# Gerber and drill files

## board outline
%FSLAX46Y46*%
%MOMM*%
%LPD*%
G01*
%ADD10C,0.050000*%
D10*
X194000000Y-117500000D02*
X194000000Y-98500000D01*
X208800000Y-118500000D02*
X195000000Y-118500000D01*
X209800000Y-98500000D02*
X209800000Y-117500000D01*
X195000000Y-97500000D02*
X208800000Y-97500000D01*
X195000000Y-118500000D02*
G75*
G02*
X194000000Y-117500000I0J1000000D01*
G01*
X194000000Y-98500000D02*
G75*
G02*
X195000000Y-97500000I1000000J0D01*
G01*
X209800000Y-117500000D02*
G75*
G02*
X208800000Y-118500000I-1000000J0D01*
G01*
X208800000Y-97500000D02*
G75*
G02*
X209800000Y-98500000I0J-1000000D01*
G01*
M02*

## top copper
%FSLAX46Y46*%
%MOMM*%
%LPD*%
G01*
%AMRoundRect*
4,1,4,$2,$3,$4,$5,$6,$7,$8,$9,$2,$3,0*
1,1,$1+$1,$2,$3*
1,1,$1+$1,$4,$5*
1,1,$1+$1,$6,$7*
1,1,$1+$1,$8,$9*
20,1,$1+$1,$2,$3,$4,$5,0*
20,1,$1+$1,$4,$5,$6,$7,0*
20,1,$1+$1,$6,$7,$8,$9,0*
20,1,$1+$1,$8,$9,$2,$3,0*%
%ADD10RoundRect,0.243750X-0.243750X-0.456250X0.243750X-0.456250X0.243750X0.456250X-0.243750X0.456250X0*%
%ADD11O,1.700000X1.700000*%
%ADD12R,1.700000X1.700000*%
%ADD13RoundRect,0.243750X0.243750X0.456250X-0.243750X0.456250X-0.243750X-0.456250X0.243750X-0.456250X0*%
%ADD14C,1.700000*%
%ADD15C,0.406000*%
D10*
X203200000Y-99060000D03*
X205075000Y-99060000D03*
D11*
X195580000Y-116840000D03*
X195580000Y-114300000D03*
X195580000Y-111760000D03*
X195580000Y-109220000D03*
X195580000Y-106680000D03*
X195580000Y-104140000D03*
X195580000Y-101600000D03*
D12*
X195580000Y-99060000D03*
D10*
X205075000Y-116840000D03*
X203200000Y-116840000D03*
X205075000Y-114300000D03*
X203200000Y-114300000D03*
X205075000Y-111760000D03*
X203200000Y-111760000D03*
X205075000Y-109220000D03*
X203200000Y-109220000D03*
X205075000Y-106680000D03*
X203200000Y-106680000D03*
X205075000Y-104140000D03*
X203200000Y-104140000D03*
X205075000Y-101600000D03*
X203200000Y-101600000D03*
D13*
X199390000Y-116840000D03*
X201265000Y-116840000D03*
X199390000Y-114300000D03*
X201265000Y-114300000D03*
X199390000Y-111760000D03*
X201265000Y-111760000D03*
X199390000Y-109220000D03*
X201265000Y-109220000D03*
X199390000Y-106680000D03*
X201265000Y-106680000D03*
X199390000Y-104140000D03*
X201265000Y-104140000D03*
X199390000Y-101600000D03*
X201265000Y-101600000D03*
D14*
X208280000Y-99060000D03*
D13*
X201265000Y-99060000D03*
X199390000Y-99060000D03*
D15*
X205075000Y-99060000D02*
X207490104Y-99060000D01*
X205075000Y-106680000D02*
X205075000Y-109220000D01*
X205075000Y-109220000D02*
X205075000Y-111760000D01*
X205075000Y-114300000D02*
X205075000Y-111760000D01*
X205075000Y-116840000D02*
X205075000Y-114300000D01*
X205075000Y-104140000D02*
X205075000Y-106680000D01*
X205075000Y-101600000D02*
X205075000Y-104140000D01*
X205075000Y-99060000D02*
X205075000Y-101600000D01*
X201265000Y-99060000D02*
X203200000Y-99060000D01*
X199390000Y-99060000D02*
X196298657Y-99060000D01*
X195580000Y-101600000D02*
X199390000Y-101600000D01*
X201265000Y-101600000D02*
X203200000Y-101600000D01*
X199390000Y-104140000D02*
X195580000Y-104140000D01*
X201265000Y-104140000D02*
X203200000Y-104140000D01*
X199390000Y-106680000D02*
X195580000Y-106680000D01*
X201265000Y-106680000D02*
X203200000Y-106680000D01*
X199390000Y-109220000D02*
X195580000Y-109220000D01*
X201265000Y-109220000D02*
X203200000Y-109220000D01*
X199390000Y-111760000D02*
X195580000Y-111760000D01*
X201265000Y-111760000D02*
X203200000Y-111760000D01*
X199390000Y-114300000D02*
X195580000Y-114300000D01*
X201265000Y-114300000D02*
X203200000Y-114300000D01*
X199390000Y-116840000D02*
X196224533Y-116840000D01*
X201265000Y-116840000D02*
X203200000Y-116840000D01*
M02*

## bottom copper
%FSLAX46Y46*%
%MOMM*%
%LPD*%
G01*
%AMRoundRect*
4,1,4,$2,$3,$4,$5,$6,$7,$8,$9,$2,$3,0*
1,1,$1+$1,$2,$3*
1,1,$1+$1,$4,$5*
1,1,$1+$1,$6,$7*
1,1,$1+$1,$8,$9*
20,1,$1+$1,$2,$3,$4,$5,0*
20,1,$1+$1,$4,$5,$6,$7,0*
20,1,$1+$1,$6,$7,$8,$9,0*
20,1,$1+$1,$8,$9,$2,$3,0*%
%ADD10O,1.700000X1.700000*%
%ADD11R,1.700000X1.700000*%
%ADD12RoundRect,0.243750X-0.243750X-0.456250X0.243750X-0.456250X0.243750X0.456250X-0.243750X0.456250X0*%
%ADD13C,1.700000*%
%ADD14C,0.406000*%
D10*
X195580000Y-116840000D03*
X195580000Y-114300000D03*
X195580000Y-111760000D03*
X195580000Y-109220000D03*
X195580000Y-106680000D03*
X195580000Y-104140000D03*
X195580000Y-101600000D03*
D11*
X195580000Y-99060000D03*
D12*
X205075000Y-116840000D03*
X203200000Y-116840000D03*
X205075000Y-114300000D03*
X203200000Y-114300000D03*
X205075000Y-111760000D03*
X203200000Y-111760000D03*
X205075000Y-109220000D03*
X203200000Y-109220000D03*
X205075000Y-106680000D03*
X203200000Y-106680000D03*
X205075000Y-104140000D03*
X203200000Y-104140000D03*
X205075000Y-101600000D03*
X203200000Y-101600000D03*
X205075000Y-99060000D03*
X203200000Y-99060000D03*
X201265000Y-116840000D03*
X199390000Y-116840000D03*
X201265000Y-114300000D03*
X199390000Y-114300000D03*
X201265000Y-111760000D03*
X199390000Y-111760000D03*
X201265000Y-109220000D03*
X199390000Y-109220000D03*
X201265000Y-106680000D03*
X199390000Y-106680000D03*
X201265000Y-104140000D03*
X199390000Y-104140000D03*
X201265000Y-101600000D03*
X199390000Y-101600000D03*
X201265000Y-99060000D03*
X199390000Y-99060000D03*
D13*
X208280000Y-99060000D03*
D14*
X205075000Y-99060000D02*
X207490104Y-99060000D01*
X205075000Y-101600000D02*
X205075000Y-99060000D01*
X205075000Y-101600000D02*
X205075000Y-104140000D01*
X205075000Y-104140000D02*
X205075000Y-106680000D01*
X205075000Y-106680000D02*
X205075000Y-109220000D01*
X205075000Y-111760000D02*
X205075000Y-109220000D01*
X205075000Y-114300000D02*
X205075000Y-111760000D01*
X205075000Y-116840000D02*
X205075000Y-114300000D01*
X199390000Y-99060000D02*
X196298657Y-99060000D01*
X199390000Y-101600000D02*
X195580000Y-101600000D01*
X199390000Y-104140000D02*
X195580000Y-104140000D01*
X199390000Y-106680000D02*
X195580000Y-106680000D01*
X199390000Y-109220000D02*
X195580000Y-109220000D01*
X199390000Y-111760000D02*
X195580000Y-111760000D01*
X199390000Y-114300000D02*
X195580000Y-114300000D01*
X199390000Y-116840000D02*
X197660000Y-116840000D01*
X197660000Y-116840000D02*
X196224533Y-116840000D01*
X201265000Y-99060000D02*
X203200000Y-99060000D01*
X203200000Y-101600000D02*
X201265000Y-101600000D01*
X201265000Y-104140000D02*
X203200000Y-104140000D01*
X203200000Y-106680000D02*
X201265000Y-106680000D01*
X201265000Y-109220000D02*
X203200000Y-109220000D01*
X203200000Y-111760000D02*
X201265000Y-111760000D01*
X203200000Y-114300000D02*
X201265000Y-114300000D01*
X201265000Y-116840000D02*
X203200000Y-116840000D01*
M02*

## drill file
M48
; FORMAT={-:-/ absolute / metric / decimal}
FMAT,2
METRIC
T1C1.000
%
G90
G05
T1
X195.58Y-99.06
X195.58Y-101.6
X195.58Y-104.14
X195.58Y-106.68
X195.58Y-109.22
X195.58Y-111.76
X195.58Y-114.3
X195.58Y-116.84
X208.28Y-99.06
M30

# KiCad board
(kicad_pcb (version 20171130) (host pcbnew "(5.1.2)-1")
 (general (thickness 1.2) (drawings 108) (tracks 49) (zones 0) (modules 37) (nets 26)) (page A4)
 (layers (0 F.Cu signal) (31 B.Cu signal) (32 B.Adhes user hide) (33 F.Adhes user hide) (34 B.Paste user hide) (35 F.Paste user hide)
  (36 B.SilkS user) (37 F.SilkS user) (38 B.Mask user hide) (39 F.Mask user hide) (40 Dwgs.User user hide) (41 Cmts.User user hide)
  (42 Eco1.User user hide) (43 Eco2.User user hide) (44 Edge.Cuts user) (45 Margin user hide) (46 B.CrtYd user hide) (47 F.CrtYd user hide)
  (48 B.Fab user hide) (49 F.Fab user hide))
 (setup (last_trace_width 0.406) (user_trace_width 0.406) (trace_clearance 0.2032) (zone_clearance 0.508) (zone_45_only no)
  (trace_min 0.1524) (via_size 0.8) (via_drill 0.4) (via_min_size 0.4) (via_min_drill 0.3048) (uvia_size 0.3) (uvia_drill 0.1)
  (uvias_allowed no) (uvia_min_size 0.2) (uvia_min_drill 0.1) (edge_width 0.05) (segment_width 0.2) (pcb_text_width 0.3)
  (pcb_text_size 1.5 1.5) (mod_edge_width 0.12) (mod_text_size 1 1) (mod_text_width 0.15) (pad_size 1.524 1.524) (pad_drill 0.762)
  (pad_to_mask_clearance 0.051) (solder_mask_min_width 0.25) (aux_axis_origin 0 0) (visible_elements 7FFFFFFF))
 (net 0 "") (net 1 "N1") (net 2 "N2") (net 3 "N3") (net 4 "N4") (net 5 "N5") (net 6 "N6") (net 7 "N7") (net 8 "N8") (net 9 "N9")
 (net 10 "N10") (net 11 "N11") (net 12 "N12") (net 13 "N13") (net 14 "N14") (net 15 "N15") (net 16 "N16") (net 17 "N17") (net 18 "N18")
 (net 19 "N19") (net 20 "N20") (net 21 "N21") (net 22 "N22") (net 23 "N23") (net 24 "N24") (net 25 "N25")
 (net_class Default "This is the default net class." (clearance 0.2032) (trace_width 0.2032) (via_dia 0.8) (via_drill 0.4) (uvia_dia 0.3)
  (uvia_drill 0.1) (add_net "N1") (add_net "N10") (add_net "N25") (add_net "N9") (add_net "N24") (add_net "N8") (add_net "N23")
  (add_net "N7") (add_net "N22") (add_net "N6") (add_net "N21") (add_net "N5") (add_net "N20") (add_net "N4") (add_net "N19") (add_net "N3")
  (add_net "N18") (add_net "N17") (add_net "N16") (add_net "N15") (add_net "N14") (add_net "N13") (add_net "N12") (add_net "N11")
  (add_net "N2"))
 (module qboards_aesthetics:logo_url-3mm (layer F.Cu) (at 208.026 116.332 90)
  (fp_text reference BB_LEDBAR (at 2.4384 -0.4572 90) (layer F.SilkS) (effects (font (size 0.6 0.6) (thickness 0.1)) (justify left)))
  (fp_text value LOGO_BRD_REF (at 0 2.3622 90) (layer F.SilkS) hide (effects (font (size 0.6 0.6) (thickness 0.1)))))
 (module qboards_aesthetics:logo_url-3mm (layer B.Cu) (at 208.026 107.442 270)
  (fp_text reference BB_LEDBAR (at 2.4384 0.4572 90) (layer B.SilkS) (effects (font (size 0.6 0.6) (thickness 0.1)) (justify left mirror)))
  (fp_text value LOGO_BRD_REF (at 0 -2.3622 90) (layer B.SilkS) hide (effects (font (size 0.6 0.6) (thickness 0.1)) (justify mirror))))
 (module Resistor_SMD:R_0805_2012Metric (layer F.Cu) (at 204.1375 99.06)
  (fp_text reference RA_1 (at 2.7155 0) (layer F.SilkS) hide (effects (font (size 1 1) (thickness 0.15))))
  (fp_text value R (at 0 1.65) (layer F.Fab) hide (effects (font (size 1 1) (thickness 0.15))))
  (pad 1 smd roundrect (at -0.9375 0) (size 0.975 1.4) (layers F.Cu F.Paste F.Mask) (roundrect_rratio 0.25) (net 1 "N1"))
  (pad 2 smd roundrect (at 0.9375 0) (size 0.975 1.4) (layers F.Cu F.Paste F.Mask) (roundrect_rratio 0.25) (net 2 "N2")))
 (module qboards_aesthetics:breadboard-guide (layer F.Cu) (at 162.56 96.52)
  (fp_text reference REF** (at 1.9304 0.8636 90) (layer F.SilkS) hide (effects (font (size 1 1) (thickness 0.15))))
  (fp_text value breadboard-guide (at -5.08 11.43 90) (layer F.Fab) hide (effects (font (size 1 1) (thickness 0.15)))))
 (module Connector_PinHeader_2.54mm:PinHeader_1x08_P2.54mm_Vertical (layer B.Cu) (at 195.58 99.06 180)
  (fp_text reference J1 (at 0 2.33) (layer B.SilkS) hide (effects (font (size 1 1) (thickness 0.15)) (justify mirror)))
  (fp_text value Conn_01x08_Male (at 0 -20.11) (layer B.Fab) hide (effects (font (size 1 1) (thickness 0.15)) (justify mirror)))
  (pad 8 thru_hole oval (at 0 -17.78 180) (size 1.7 1.7) (drill 1) (layers *.Cu *.Mask) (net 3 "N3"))
  (pad 7 thru_hole oval (at 0 -15.24 180) (size 1.7 1.7) (drill 1) (layers *.Cu *.Mask) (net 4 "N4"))
  (pad 6 thru_hole oval (at 0 -12.7 180) (size 1.7 1.7) (drill 1) (layers *.Cu *.Mask) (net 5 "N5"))
  (pad 5 thru_hole oval (at 0 -10.16 180) (size 1.7 1.7) (drill 1) (layers *.Cu *.Mask) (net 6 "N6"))
  (pad 4 thru_hole oval (at 0 -7.62 180) (size 1.7 1.7) (drill 1) (layers *.Cu *.Mask) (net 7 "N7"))
  (pad 3 thru_hole oval (at 0 -5.08 180) (size 1.7 1.7) (drill 1) (layers *.Cu *.Mask) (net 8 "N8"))
  (pad 2 thru_hole oval (at 0 -2.54 180) (size 1.7 1.7) (drill 1) (layers *.Cu *.Mask) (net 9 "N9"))
  (pad 1 thru_hole rect (at 0 0 180) (size 1.7 1.7) (drill 1) (layers *.Cu *.Mask) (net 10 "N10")))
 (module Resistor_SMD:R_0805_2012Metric (layer B.Cu) (at 204.1375 116.84)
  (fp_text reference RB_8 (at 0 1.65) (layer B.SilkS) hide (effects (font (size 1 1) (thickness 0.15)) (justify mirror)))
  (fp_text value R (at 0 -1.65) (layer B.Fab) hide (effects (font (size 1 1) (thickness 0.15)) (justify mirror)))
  (pad 2 smd roundrect (at 0.9375 0) (size 0.975 1.4) (layers B.Cu B.Paste B.Mask) (roundrect_rratio 0.25) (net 2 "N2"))
  (pad 1 smd roundrect (at -0.9375 0) (size 0.975 1.4) (layers B.Cu B.Paste B.Mask) (roundrect_rratio 0.25) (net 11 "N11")))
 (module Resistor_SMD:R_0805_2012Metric (layer B.Cu) (at 204.1375 114.3)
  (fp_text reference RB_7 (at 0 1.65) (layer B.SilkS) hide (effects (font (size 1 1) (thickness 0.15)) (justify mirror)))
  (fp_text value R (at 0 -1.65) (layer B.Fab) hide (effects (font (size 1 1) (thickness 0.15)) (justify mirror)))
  (pad 2 smd roundrect (at 0.9375 0) (size 0.975 1.4) (layers B.Cu B.Paste B.Mask) (roundrect_rratio 0.25) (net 2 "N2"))
  (pad 1 smd roundrect (at -0.9375 0) (size 0.975 1.4) (layers B.Cu B.Paste B.Mask) (roundrect_rratio 0.25) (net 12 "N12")))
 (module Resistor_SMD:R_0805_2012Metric (layer B.Cu) (at 204.1375 111.76)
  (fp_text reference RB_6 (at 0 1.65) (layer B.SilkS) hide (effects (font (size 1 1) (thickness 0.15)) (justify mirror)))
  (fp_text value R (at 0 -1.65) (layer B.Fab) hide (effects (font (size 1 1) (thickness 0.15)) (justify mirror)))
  (pad 2 smd roundrect (at 0.9375 0) (size 0.975 1.4) (layers B.Cu B.Paste B.Mask) (roundrect_rratio 0.25) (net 2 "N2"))
  (pad 1 smd roundrect (at -0.9375 0) (size 0.975 1.4) (layers B.Cu B.Paste B.Mask) (roundrect_rratio 0.25) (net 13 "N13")))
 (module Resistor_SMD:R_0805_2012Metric (layer B.Cu) (at 204.1375 109.22)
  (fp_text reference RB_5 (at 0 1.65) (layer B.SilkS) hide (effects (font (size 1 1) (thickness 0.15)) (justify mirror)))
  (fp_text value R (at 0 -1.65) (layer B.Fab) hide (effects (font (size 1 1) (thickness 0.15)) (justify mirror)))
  (pad 2 smd roundrect (at 0.9375 0) (size 0.975 1.4) (layers B.Cu B.Paste B.Mask) (roundrect_rratio 0.25) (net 2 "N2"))
  (pad 1 smd roundrect (at -0.9375 0) (size 0.975 1.4) (layers B.Cu B.Paste B.Mask) (roundrect_rratio 0.25) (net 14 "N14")))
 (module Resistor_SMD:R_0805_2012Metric (layer B.Cu) (at 204.1375 106.68)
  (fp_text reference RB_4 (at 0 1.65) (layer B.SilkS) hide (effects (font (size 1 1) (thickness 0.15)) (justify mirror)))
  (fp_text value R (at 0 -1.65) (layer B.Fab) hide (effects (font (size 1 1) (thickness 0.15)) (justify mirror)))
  (pad 2 smd roundrect (at 0.9375 0) (size 0.975 1.4) (layers B.Cu B.Paste B.Mask) (roundrect_rratio 0.25) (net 2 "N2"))
  (pad 1 smd roundrect (at -0.9375 0) (size 0.975 1.4) (layers B.Cu B.Paste B.Mask) (roundrect_rratio 0.25) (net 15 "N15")))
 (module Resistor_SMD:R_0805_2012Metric (layer B.Cu) (at 204.1375 104.14)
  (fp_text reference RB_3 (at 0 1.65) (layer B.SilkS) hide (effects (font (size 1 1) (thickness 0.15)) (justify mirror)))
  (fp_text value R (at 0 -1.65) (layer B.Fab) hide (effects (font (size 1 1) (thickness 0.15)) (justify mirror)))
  (pad 2 smd roundrect (at 0.9375 0) (size 0.975 1.4) (layers B.Cu B.Paste B.Mask) (roundrect_rratio 0.25) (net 2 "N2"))
  (pad 1 smd roundrect (at -0.9375 0) (size 0.975 1.4) (layers B.Cu B.Paste B.Mask) (roundrect_rratio 0.25) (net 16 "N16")))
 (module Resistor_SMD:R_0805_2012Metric (layer B.Cu) (at 204.1375 101.6)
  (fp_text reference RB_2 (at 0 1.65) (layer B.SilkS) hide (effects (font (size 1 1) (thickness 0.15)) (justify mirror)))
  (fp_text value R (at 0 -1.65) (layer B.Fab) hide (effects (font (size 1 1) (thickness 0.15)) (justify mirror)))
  (pad 2 smd roundrect (at 0.9375 0) (size 0.975 1.4) (layers B.Cu B.Paste B.Mask) (roundrect_rratio 0.25) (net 2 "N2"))
  (pad 1 smd roundrect (at -0.9375 0) (size 0.975 1.4) (layers B.Cu B.Paste B.Mask) (roundrect_rratio 0.25) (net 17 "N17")))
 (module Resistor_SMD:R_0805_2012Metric (layer B.Cu) (at 204.1375 99.06)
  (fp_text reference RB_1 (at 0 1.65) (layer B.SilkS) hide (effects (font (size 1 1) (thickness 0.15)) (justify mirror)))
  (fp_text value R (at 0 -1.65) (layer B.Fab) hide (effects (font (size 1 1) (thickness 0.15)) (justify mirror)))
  (pad 2 smd roundrect (at 0.9375 0) (size 0.975 1.4) (layers B.Cu B.Paste B.Mask) (roundrect_rratio 0.25) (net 2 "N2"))
  (pad 1 smd roundrect (at -0.9375 0) (size 0.975 1.4) (layers B.Cu B.Paste B.Mask) (roundrect_rratio 0.25) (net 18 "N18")))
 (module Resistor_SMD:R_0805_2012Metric (layer F.Cu) (at 204.1375 116.84)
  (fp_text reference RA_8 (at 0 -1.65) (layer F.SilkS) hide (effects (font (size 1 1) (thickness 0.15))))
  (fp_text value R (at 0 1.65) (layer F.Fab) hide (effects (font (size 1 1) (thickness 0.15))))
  (pad 2 smd roundrect (at 0.9375 0) (size 0.975 1.4) (layers F.Cu F.Paste F.Mask) (roundrect_rratio 0.25) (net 2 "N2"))
  (pad 1 smd roundrect (at -0.9375 0) (size 0.975 1.4) (layers F.Cu F.Paste F.Mask) (roundrect_rratio 0.25) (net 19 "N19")))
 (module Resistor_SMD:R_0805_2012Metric (layer F.Cu) (at 204.1375 114.3)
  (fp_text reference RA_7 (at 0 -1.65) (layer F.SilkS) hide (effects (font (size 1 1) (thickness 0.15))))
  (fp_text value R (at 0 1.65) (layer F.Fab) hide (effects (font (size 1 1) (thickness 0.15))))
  (pad 2 smd roundrect (at 0.9375 0) (size 0.975 1.4) (layers F.Cu F.Paste F.Mask) (roundrect_rratio 0.25) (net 2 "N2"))
  (pad 1 smd roundrect (at -0.9375 0) (size 0.975 1.4) (layers F.Cu F.Paste F.Mask) (roundrect_rratio 0.25) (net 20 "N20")))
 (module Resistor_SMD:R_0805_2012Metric (layer F.Cu) (at 204.1375 111.76)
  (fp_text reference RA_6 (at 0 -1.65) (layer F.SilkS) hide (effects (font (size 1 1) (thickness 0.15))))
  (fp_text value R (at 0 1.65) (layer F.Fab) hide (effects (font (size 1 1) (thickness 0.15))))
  (pad 2 smd roundrect (at 0.9375 0) (size 0.975 1.4) (layers F.Cu F.Paste F.Mask) (roundrect_rratio 0.25) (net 2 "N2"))
  (pad 1 smd roundrect (at -0.9375 0) (size 0.975 1.4) (layers F.Cu F.Paste F.Mask) (roundrect_rratio 0.25) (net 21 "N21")))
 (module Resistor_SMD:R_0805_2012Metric (layer F.Cu) (at 204.1375 109.22)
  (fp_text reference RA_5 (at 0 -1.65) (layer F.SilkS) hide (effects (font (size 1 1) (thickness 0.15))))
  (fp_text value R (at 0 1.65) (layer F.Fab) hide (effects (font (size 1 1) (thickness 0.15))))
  (pad 2 smd roundrect (at 0.9375 0) (size 0.975 1.4) (layers F.Cu F.Paste F.Mask) (roundrect_rratio 0.25) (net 2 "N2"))
  (pad 1 smd roundrect (at -0.9375 0) (size 0.975 1.4) (layers F.Cu F.Paste F.Mask) (roundrect_rratio 0.25) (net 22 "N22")))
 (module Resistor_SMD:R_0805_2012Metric (layer F.Cu) (at 204.1375 106.68)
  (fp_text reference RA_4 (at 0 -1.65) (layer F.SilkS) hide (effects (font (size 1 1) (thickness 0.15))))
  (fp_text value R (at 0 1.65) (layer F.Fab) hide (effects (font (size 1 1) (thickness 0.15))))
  (pad 2 smd roundrect (at 0.9375 0) (size 0.975 1.4) (layers F.Cu F.Paste F.Mask) (roundrect_rratio 0.25) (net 2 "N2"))
  (pad 1 smd roundrect (at -0.9375 0) (size 0.975 1.4) (layers F.Cu F.Paste F.Mask) (roundrect_rratio 0.25) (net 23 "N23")))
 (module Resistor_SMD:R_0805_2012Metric (layer F.Cu) (at 204.1375 104.14)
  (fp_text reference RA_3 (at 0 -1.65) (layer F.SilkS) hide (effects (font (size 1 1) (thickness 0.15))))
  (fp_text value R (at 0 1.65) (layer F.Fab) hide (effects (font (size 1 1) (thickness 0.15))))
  (pad 2 smd roundrect (at 0.9375 0) (size 0.975 1.4) (layers F.Cu F.Paste F.Mask) (roundrect_rratio 0.25) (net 2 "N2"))
  (pad 1 smd roundrect (at -0.9375 0) (size 0.975 1.4) (layers F.Cu F.Paste F.Mask) (roundrect_rratio 0.25) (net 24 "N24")))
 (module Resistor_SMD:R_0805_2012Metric (layer F.Cu) (at 204.1375 101.6)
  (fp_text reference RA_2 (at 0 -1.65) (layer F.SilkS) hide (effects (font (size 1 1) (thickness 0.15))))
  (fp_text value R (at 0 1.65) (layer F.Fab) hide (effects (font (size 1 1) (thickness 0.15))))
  (pad 2 smd roundrect (at 0.9375 0) (size 0.975 1.4) (layers F.Cu F.Paste F.Mask) (roundrect_rratio 0.25) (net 2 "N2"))
  (pad 1 smd roundrect (at -0.9375 0) (size 0.975 1.4) (layers F.Cu F.Paste F.Mask) (roundrect_rratio 0.25) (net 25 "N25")))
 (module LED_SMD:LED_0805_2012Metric (layer B.Cu) (at 200.3275 116.84)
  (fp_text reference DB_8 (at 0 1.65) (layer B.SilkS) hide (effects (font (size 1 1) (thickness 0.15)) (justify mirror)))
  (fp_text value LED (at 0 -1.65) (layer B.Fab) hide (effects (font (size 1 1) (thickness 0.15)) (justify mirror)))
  (pad 2 smd roundrect (at 0.9375 0) (size 0.975 1.4) (layers B.Cu B.Paste B.Mask) (roundrect_rratio 0.25) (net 11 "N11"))
  (pad 1 smd roundrect (at -0.9375 0) (size 0.975 1.4) (layers B.Cu B.Paste B.Mask) (roundrect_rratio 0.25) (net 3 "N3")))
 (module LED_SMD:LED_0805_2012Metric (layer B.Cu) (at 200.3275 114.3)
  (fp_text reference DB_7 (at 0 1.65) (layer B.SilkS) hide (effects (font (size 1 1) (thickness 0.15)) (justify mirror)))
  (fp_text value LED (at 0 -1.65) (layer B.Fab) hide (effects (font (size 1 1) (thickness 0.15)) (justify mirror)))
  (pad 2 smd roundrect (at 0.9375 0) (size 0.975 1.4) (layers B.Cu B.Paste B.Mask) (roundrect_rratio 0.25) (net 12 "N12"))
  (pad 1 smd roundrect (at -0.9375 0) (size 0.975 1.4) (layers B.Cu B.Paste B.Mask) (roundrect_rratio 0.25) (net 4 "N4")))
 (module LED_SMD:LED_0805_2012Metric (layer B.Cu) (at 200.3275 111.76)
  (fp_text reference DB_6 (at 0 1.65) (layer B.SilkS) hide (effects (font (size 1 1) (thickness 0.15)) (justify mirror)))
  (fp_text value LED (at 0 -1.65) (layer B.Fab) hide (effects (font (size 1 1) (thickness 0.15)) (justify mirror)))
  (pad 2 smd roundrect (at 0.9375 0) (size 0.975 1.4) (layers B.Cu B.Paste B.Mask) (roundrect_rratio 0.25) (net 13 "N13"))
  (pad 1 smd roundrect (at -0.9375 0) (size 0.975 1.4) (layers B.Cu B.Paste B.Mask) (roundrect_rratio 0.25) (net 5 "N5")))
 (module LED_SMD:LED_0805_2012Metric (layer B.Cu) (at 200.3275 109.22)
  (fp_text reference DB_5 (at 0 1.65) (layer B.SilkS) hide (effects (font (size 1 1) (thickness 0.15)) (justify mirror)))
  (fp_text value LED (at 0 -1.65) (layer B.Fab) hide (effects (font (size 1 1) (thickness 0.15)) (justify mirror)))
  (pad 2 smd roundrect (at 0.9375 0) (size 0.975 1.4) (layers B.Cu B.Paste B.Mask) (roundrect_rratio 0.25) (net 14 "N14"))
  (pad 1 smd roundrect (at -0.9375 0) (size 0.975 1.4) (layers B.Cu B.Paste B.Mask) (roundrect_rratio 0.25) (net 6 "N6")))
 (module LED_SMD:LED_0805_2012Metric (layer B.Cu) (at 200.3275 106.68)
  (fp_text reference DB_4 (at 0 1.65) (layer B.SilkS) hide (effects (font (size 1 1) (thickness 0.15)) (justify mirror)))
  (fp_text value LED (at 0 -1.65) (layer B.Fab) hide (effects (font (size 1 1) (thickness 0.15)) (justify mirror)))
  (pad 2 smd roundrect (at 0.9375 0) (size 0.975 1.4) (layers B.Cu B.Paste B.Mask) (roundrect_rratio 0.25) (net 15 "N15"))
  (pad 1 smd roundrect (at -0.9375 0) (size 0.975 1.4) (layers B.Cu B.Paste B.Mask) (roundrect_rratio 0.25) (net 7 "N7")))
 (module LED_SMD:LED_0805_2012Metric (layer B.Cu) (at 200.3275 104.14)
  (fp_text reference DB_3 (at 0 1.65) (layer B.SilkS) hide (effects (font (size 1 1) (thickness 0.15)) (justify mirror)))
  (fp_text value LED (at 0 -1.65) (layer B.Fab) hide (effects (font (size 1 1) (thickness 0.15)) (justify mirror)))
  (pad 2 smd roundrect (at 0.9375 0) (size 0.975 1.4) (layers B.Cu B.Paste B.Mask) (roundrect_rratio 0.25) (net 16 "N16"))
  (pad 1 smd roundrect (at -0.9375 0) (size 0.975 1.4) (layers B.Cu B.Paste B.Mask) (roundrect_rratio 0.25) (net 8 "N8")))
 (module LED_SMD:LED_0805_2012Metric (layer B.Cu) (at 200.3275 101.6)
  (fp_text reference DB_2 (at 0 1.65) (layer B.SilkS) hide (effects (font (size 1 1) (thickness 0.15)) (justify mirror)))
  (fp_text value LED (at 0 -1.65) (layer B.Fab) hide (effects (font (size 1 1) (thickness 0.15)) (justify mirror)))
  (pad 2 smd roundrect (at 0.9375 0) (size 0.975 1.4) (layers B.Cu B.Paste B.Mask) (roundrect_rratio 0.25) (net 17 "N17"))
  (pad 1 smd roundrect (at -0.9375 0) (size 0.975 1.4) (layers B.Cu B.Paste B.Mask) (roundrect_rratio 0.25) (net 9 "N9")))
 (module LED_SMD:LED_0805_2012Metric (layer B.Cu) (at 200.3275 99.06)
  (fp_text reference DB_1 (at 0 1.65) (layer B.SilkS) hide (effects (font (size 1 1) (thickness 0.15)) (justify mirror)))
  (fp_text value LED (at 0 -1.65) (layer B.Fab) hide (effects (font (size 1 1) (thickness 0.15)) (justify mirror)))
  (pad 2 smd roundrect (at 0.9375 0) (size 0.975 1.4) (layers B.Cu B.Paste B.Mask) (roundrect_rratio 0.25) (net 18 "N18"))
  (pad 1 smd roundrect (at -0.9375 0) (size 0.975 1.4) (layers B.Cu B.Paste B.Mask) (roundrect_rratio 0.25) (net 10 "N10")))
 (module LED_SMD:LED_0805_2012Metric (layer F.Cu) (at 200.3275 116.84 180)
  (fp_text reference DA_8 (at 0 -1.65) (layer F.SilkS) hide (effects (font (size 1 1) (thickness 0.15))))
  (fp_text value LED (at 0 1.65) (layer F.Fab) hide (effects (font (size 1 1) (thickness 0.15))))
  (pad 2 smd roundrect (at 0.9375 0 180) (size 0.975 1.4) (layers F.Cu F.Paste F.Mask) (roundrect_rratio 0.25) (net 3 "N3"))
  (pad 1 smd roundrect (at -0.9375 0 180) (size 0.975 1.4) (layers F.Cu F.Paste F.Mask) (roundrect_rratio 0.25) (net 19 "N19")))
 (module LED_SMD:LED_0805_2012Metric (layer F.Cu) (at 200.3275 114.3 180)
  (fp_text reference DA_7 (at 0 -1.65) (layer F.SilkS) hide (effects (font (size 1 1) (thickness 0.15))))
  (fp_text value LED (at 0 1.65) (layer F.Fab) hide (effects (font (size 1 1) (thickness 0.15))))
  (pad 2 smd roundrect (at 0.9375 0 180) (size 0.975 1.4) (layers F.Cu F.Paste F.Mask) (roundrect_rratio 0.25) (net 4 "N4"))
  (pad 1 smd roundrect (at -0.9375 0 180) (size 0.975 1.4) (layers F.Cu F.Paste F.Mask) (roundrect_rratio 0.25) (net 20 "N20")))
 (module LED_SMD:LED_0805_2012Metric (layer F.Cu) (at 200.3275 111.76 180)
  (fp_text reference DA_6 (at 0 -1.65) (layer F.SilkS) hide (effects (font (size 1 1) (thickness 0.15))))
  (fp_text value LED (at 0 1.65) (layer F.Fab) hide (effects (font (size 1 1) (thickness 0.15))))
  (pad 2 smd roundrect (at 0.9375 0 180) (size 0.975 1.4) (layers F.Cu F.Paste F.Mask) (roundrect_rratio 0.25) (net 5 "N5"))
  (pad 1 smd roundrect (at -0.9375 0 180) (size 0.975 1.4) (layers F.Cu F.Paste F.Mask) (roundrect_rratio 0.25) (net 21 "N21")))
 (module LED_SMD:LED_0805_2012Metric (layer F.Cu) (at 200.3275 109.22 180)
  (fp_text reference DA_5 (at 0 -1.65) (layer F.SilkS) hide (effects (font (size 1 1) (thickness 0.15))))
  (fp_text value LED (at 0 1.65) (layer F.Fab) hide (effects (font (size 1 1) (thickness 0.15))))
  (pad 2 smd roundrect (at 0.9375 0 180) (size 0.975 1.4) (layers F.Cu F.Paste F.Mask) (roundrect_rratio 0.25) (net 6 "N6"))
  (pad 1 smd roundrect (at -0.9375 0 180) (size 0.975 1.4) (layers F.Cu F.Paste F.Mask) (roundrect_rratio 0.25) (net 22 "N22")))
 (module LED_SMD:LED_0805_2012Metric (layer F.Cu) (at 200.3275 106.68 180)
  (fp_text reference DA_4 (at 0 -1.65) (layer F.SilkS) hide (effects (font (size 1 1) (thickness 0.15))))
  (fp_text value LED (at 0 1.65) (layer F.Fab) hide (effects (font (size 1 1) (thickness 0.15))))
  (pad 2 smd roundrect (at 0.9375 0 180) (size 0.975 1.4) (layers F.Cu F.Paste F.Mask) (roundrect_rratio 0.25) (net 7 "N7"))
  (pad 1 smd roundrect (at -0.9375 0 180) (size 0.975 1.4) (layers F.Cu F.Paste F.Mask) (roundrect_rratio 0.25) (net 23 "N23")))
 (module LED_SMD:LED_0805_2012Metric (layer F.Cu) (at 200.3275 104.14 180)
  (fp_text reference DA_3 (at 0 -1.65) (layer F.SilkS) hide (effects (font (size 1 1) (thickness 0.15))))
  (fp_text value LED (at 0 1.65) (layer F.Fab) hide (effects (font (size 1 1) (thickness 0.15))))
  (pad 2 smd roundrect (at 0.9375 0 180) (size 0.975 1.4) (layers F.Cu F.Paste F.Mask) (roundrect_rratio 0.25) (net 8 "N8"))
  (pad 1 smd roundrect (at -0.9375 0 180) (size 0.975 1.4) (layers F.Cu F.Paste F.Mask) (roundrect_rratio 0.25) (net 24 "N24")))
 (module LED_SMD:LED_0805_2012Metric (layer F.Cu) (at 200.3275 101.6 180)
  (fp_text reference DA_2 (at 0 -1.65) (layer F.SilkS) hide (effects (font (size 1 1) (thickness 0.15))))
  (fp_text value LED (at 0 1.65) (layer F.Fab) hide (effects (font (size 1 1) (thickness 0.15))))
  (pad 2 smd roundrect (at 0.9375 0 180) (size 0.975 1.4) (layers F.Cu F.Paste F.Mask) (roundrect_rratio 0.25) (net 9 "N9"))
  (pad 1 smd roundrect (at -0.9375 0 180) (size 0.975 1.4) (layers F.Cu F.Paste F.Mask) (roundrect_rratio 0.25) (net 25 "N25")))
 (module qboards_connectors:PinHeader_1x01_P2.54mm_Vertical (layer F.Cu) (at 208.28 99.06 90)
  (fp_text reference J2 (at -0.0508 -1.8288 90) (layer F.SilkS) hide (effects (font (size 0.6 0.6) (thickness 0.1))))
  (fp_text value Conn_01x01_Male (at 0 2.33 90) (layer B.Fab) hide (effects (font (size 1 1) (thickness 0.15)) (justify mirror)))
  (pad 1 thru_hole circle (at 0 0 90) (size 1.7 1.7) (drill 1) (layers *.Cu *.Mask) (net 2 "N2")))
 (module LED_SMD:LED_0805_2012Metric (layer F.Cu) (at 200.3275 99.06 180)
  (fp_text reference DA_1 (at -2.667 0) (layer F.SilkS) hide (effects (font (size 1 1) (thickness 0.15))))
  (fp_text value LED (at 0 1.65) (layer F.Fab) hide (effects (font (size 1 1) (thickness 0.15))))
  (pad 1 smd roundrect (at -0.9375 0 180) (size 0.975 1.4) (layers F.Cu F.Paste F.Mask) (roundrect_rratio 0.25) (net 1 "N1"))
  (pad 2 smd roundrect (at 0.9375 0 180) (size 0.975 1.4) (layers F.Cu F.Paste F.Mask) (roundrect_rratio 0.25) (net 10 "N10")))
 (gr_line (start 194 117.5) (end 194 98.5) (layer Edge.Cuts) (width 0.05))
 (gr_line (start 208.8 118.5) (end 195 118.5) (layer Edge.Cuts) (width 0.05))
 (gr_line (start 209.8 98.5) (end 209.8 117.5) (layer Edge.Cuts) (width 0.05))
 (gr_line (start 195 97.5) (end 208.8 97.5) (layer Edge.Cuts) (width 0.05))
 (gr_arc (start 195 117.5) (end 194 117.5) (angle -90) (layer Edge.Cuts) (width 0.05))
 (gr_arc (start 195 98.5) (end 195 97.5) (angle -90) (layer Edge.Cuts) (width 0.05))
 (gr_arc (start 208.8 117.5) (end 208.8 118.5) (angle -90) (layer Edge.Cuts) (width 0.05))
 (gr_arc (start 208.8 98.5) (end 209.8 98.5) (angle -90) (layer Edge.Cuts) (width 0.05))
 (segment (start 205.075 99.06) (end 207.490104 99.06) (width 0.406) (layer F.Cu) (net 2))
 (segment (start 205.075 106.68) (end 205.075 109.22) (width 0.406) (layer F.Cu) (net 2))
 (segment (start 205.075 109.22) (end 205.075 111.76) (width 0.406) (layer F.Cu) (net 2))
 (segment (start 205.075 114.3) (end 205.075 111.76) (width 0.406) (layer F.Cu) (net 2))
 (segment (start 205.075 116.84) (end 205.075 114.3) (width 0.406) (layer F.Cu) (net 2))
 (segment (start 205.075 99.06) (end 207.490104 99.06) (width 0.406) (layer B.Cu) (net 2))
 (segment (start 205.075 104.14) (end 205.075 106.68) (width 0.406) (layer F.Cu) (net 2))
 (segment (start 205.075 101.6) (end 205.075 104.14) (width 0.406) (layer F.Cu) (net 2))
 (segment (start 205.075 99.06) (end 205.075 101.6) (width 0.406) (layer F.Cu) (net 2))
 (segment (start 205.075 101.6) (end 205.075 99.06) (width 0.406) (layer B.Cu) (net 2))
 (segment (start 205.075 101.6) (end 205.075 104.14) (width 0.406) (layer B.Cu) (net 2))
 (segment (start 205.075 104.14) (end 205.075 106.68) (width 0.406) (layer B.Cu) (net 2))
 (segment (start 205.075 106.68) (end 205.075 109.22) (width 0.406) (layer B.Cu) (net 2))
 (segment (start 205.075 111.76) (end 205.075 109.22) (width 0.406) (layer B.Cu) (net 2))
 (segment (start 205.075 114.3) (end 205.075 111.76) (width 0.406) (layer B.Cu) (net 2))
 (segment (start 205.075 116.84) (end 205.075 114.3) (width 0.406) (layer B.Cu) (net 2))
 (segment (start 201.265 99.06) (end 203.2 99.06) (width 0.406) (layer F.Cu) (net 1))
 (segment (start 199.39 99.06) (end 196.298657 99.06) (width 0.406) (layer B.Cu) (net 10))
 (segment (start 199.39 99.06) (end 196.298657 99.06) (width 0.406) (layer F.Cu) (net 10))
 (segment (start 195.58 101.6) (end 199.39 101.6) (width 0.406) (layer F.Cu) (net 9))
 (segment (start 199.39 101.6) (end 195.58 101.6) (width 0.406) (layer B.Cu) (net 9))
 (segment (start 201.265 101.6) (end 203.2 101.6) (width 0.406) (layer F.Cu) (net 25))
 (segment (start 199.39 104.14) (end 195.58 104.14) (width 0.406) (layer F.Cu) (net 8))
 (segment (start 199.39 104.14) (end 195.58 104.14) (width 0.406) (layer B.Cu) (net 8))
 (segment (start 201.265 104.14) (end 203.2 104.14) (width 0.406) (layer F.Cu) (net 24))
 (segment (start 199.39 106.68) (end 195.58 106.68) (width 0.406) (layer F.Cu) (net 7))
 (segment (start 199.39 106.68) (end 195.58 106.68) (width 0.406) (layer B.Cu) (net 7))
 (segment (start 201.265 106.68) (end 203.2 106.68) (width 0.406) (layer F.Cu) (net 23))
 (segment (start 199.39 109.22) (end 195.58 109.22) (width 0.406) (layer F.Cu) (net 6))
 (segment (start 199.39 109.22) (end 195.58 109.22) (width 0.406) (layer B.Cu) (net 6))
 (segment (start 201.265 109.22) (end 203.2 109.22) (width 0.406) (layer F.Cu) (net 22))
 (segment (start 199.39 111.76) (end 195.58 111.76) (width 0.406) (layer F.Cu) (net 5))
 (segment (start 199.39 111.76) (end 195.58 111.76) (width 0.406) (layer B.Cu) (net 5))
 (segment (start 201.265 111.76) (end 203.2 111.76) (width 0.406) (layer F.Cu) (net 21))
 (segment (start 199.39 114.3) (end 195.58 114.3) (width 0.406) (layer F.Cu) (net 4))
 (segment (start 199.39 114.3) (end 195.58 114.3) (width 0.406) (layer B.Cu) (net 4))
 (segment (start 201.265 114.3) (end 203.2 114.3) (width 0.406) (layer F.Cu) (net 20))
 (segment (start 199.39 116.84) (end 196.224533 116.84) (width 0.406) (layer F.Cu) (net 3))
 (segment (start 199.39 116.84) (end 197.66 116.84) (width 0.406) (layer B.Cu) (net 3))
 (segment (start 197.66 116.84) (end 196.224533 116.84) (width 0.406) (layer B.Cu) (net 3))
 (segment (start 201.265 116.84) (end 203.2 116.84) (width 0.406) (layer F.Cu) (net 19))
 (segment (start 201.265 99.06) (end 203.2 99.06) (width 0.406) (layer B.Cu) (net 18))
 (segment (start 203.2 101.6) (end 201.265 101.6) (width 0.406) (layer B.Cu) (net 17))
 (segment (start 201.265 104.14) (end 203.2 104.14) (width 0.406) (layer B.Cu) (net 16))
 (segment (start 203.2 106.68) (end 201.265 106.68) (width 0.406) (layer B.Cu) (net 15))
 (segment (start 201.265 109.22) (end 203.2 109.22) (width 0.406) (layer B.Cu) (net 14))
 (segment (start 203.2 111.76) (end 201.265 111.76) (width 0.406) (layer B.Cu) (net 13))
 (segment (start 203.2 114.3) (end 201.265 114.3) (width 0.406) (layer B.Cu) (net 12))
 (segment (start 201.265 116.84) (end 203.2 116.84) (width 0.406) (layer B.Cu) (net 11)))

